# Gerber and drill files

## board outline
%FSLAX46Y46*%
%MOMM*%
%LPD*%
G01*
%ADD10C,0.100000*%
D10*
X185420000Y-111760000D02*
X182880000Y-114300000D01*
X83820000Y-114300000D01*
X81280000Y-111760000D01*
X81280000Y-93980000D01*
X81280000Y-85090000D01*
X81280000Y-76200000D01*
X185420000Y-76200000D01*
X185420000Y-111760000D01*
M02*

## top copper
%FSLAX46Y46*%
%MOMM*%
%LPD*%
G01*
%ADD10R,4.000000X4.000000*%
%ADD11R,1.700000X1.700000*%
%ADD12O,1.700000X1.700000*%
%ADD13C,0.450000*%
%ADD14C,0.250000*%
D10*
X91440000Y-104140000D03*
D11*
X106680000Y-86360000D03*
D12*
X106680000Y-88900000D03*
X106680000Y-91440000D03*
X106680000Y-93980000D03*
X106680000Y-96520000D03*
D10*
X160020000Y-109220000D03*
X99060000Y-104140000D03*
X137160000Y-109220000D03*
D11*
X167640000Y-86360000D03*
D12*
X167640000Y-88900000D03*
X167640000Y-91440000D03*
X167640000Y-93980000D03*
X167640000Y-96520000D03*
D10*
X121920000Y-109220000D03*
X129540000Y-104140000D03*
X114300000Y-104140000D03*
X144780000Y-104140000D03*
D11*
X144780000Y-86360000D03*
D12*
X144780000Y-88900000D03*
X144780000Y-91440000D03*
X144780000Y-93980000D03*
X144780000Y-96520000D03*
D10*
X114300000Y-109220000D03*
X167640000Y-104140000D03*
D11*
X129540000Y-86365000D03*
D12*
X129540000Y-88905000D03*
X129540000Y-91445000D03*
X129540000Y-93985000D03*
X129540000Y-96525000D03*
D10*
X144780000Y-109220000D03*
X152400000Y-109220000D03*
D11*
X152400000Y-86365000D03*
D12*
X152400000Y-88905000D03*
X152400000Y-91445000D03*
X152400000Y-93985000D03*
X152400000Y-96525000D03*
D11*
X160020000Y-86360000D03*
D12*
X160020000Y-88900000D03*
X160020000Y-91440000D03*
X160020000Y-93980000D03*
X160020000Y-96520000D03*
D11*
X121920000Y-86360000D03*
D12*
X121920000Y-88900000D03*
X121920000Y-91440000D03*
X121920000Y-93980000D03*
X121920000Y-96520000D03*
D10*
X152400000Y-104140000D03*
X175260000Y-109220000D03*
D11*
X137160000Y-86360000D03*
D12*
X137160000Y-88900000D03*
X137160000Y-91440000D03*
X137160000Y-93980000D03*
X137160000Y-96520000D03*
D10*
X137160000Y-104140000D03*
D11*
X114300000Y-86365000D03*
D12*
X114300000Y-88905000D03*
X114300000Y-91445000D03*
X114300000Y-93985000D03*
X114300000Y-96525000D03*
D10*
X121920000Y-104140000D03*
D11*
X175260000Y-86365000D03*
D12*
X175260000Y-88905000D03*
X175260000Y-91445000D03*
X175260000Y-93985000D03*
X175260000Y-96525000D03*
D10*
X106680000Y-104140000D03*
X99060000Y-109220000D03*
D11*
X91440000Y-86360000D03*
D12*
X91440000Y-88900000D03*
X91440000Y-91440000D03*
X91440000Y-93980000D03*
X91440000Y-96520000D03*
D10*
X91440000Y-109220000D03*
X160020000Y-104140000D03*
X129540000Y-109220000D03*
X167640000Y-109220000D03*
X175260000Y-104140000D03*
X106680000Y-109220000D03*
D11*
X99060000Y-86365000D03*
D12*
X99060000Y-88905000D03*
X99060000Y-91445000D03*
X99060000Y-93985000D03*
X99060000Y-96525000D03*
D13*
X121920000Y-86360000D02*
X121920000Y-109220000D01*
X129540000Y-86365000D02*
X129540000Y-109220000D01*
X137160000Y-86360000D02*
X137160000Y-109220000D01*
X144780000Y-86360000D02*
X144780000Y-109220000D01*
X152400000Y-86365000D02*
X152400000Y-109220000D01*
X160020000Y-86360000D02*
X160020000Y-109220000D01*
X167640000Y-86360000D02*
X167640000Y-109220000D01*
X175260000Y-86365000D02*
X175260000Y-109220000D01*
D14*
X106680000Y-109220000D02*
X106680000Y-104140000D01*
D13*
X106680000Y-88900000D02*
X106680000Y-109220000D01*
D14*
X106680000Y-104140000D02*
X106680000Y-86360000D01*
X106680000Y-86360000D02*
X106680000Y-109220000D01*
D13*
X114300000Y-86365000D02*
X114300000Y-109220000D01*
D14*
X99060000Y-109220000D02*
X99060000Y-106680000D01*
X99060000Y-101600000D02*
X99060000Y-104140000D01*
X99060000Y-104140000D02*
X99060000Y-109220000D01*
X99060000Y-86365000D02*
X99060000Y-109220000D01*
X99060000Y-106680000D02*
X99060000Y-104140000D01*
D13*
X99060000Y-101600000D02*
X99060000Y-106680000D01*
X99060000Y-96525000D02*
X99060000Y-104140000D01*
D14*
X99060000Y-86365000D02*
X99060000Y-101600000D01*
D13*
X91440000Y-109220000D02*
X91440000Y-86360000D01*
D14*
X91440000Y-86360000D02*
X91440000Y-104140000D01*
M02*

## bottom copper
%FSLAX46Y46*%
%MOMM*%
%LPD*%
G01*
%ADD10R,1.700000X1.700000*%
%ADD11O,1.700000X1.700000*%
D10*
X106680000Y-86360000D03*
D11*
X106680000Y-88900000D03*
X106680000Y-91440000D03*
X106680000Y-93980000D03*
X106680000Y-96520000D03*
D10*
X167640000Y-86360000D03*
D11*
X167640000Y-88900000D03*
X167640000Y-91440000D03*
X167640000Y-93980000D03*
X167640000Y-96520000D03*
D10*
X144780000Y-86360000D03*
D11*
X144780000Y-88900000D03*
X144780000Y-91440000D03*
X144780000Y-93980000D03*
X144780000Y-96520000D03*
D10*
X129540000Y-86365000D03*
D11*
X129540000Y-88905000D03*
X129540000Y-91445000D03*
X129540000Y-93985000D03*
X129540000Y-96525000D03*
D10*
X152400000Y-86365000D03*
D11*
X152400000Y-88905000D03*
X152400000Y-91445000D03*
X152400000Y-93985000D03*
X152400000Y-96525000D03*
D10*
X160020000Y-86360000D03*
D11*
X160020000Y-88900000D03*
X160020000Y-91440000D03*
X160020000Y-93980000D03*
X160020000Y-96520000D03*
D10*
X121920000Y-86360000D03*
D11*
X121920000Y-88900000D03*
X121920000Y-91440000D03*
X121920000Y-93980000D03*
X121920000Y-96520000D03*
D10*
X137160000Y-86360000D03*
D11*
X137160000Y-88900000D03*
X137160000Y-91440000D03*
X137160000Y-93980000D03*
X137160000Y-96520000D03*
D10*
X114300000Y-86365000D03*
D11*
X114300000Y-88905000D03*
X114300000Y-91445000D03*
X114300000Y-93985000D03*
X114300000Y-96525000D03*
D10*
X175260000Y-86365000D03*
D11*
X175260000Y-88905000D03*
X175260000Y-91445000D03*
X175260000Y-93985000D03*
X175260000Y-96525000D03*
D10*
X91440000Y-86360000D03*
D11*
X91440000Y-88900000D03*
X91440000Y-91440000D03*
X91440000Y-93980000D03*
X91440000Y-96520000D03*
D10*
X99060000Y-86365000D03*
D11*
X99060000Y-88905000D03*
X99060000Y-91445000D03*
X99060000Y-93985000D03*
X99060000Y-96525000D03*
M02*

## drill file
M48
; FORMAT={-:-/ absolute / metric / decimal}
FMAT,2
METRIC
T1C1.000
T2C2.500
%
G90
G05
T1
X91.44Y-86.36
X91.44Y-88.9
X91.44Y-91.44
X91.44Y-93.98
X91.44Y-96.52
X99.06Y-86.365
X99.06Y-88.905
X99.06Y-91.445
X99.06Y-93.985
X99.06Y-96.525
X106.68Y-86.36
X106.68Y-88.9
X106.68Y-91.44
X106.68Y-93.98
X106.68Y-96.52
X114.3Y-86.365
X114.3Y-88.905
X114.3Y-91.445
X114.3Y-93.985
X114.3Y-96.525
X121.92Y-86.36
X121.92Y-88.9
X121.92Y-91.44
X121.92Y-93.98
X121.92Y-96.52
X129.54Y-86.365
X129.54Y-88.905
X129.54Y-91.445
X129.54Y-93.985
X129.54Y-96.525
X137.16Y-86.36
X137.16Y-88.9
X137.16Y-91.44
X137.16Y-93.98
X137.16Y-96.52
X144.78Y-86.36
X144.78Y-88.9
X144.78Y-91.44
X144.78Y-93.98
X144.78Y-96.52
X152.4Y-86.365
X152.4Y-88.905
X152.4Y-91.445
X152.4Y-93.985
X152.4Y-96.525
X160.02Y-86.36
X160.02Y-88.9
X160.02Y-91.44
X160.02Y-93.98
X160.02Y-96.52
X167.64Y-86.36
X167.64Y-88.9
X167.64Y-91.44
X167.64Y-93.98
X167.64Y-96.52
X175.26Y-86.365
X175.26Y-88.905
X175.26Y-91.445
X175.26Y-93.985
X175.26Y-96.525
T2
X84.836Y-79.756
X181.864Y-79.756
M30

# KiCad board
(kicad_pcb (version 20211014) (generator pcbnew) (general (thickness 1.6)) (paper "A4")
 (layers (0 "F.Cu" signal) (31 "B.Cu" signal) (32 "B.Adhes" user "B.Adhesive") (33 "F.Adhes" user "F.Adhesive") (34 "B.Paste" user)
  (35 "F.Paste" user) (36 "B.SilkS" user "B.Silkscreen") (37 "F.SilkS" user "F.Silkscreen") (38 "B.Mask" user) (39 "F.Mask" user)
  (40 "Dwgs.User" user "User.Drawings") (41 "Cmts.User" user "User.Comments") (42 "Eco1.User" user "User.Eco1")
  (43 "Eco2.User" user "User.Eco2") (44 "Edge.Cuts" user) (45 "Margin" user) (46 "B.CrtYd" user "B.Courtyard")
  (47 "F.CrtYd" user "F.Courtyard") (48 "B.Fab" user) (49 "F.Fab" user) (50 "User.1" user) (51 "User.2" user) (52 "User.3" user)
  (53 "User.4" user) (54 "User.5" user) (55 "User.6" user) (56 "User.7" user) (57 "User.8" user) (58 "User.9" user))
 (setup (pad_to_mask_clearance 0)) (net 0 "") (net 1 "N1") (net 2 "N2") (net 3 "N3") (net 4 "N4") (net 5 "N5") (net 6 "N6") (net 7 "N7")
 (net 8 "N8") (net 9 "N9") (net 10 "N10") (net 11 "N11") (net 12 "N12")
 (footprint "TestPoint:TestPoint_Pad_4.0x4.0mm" (layer "F.Cu") (at 91.44 104.14 -90)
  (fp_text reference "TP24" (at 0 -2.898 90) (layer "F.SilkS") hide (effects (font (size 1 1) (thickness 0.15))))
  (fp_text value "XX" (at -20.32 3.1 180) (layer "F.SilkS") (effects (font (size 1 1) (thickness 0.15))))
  (pad "1" smd rect (at 0 0 270) (size 4 4) (layers "F.Cu" "F.Mask") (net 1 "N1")))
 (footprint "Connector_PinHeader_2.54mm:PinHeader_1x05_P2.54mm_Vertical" (layer "F.Cu") (at 106.68 86.36)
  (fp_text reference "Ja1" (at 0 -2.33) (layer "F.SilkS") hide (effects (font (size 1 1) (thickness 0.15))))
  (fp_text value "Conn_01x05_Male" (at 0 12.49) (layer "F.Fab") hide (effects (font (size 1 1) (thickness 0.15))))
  (pad "1" thru_hole rect (at 0 0) (size 1.7 1.7) (drill 1) (layers *.Cu *.Mask) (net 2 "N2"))
  (pad "2" thru_hole oval (at 0 2.54) (size 1.7 1.7) (drill 1) (layers *.Cu *.Mask) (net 2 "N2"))
  (pad "3" thru_hole oval (at 0 5.08) (size 1.7 1.7) (drill 1) (layers *.Cu *.Mask) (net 2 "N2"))
  (pad "4" thru_hole oval (at 0 7.62) (size 1.7 1.7) (drill 1) (layers *.Cu *.Mask) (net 2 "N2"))
  (pad "5" thru_hole oval (at 0 10.16) (size 1.7 1.7) (drill 1) (layers *.Cu *.Mask) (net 2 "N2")))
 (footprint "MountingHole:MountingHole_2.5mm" (layer "F.Cu") (at 84.836 79.756)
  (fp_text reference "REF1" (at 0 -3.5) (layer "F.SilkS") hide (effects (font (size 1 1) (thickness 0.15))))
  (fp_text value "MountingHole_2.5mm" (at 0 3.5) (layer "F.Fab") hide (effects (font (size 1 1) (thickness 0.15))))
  (pad "" np_thru_hole circle (at 0 0) (size 2.5 2.5) (drill 2.5) (layers *.Cu *.Mask)))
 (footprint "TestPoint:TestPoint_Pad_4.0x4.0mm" (layer "F.Cu") (at 160.02 109.22)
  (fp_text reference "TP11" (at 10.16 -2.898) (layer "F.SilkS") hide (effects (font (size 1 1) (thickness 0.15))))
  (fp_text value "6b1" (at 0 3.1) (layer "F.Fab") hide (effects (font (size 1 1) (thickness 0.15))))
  (pad "1" smd rect (at 0 0) (size 4 4) (layers "F.Cu" "F.Mask") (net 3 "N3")))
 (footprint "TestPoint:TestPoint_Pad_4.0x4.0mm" (layer "F.Cu") (at 99.06 104.14 -90)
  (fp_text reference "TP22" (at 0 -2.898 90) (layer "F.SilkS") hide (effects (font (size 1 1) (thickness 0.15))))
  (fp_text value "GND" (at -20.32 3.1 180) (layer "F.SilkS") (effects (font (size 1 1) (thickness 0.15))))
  (pad "1" smd rect (at 0 0 270) (size 4 4) (layers "F.Cu" "F.Mask") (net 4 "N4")))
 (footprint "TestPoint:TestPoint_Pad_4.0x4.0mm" (layer "F.Cu") (at 137.16 109.22)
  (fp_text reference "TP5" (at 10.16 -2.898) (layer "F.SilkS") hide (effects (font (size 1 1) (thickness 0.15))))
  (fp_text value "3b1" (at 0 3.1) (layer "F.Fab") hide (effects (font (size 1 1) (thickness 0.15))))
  (pad "1" smd rect (at 0 0) (size 4 4) (layers "F.Cu" "F.Mask") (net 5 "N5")))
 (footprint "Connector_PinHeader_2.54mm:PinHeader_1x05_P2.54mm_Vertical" (layer "F.Cu") (at 167.64 86.36)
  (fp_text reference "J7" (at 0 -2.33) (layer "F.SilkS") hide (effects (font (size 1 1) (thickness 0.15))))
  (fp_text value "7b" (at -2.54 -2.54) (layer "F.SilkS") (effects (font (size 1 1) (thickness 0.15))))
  (pad "1" thru_hole rect (at 0 0) (size 1.7 1.7) (drill 1) (layers *.Cu *.Mask) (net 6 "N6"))
  (pad "2" thru_hole oval (at 0 2.54) (size 1.7 1.7) (drill 1) (layers *.Cu *.Mask) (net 6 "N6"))
  (pad "3" thru_hole oval (at 0 5.08) (size 1.7 1.7) (drill 1) (layers *.Cu *.Mask) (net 6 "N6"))
  (pad "4" thru_hole oval (at 0 7.62) (size 1.7 1.7) (drill 1) (layers *.Cu *.Mask) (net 6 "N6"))
  (pad "5" thru_hole oval (at 0 10.16) (size 1.7 1.7) (drill 1) (layers *.Cu *.Mask) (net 6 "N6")))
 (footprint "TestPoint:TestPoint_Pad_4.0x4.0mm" (layer "F.Cu") (at 121.92 109.22)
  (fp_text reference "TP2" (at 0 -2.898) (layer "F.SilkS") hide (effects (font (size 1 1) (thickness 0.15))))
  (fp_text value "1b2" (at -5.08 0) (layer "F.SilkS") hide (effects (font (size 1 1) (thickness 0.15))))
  (pad "1" smd rect (at 0 0) (size 4 4) (layers "F.Cu" "F.Mask") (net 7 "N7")))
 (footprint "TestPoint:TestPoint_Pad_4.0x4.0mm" (layer "F.Cu") (at 129.54 104.14)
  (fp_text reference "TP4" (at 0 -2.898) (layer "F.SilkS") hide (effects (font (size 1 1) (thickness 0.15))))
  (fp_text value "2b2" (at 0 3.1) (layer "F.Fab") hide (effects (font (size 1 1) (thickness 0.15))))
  (pad "1" smd rect (at 0 0) (size 4 4) (layers "F.Cu" "F.Mask") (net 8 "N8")))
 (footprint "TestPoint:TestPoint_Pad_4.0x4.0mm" (layer "F.Cu") (at 114.3 104.14 -90)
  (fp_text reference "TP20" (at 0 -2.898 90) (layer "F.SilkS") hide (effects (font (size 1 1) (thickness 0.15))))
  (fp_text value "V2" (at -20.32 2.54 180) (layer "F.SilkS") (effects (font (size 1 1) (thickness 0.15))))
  (pad "1" smd rect (at 0 0 270) (size 4 4) (layers "F.Cu" "F.Mask") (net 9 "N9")))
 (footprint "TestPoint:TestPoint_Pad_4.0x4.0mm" (layer "F.Cu") (at 144.78 104.14)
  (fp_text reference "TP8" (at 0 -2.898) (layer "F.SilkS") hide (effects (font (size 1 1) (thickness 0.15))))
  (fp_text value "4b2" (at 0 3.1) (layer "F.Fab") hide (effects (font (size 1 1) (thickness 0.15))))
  (pad "1" smd rect (at 0 0) (size 4 4) (layers "F.Cu" "F.Mask") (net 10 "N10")))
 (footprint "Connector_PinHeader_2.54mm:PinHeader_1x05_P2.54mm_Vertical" (layer "F.Cu") (at 144.78 86.36)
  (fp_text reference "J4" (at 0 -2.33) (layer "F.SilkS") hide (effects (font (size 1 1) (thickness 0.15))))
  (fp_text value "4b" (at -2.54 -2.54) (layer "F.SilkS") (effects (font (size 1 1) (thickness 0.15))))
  (pad "1" thru_hole rect (at 0 0) (size 1.7 1.7) (drill 1) (layers *.Cu *.Mask) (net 10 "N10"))
  (pad "2" thru_hole oval (at 0 2.54) (size 1.7 1.7) (drill 1) (layers *.Cu *.Mask) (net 10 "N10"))
  (pad "3" thru_hole oval (at 0 5.08) (size 1.7 1.7) (drill 1) (layers *.Cu *.Mask) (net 10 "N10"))
  (pad "4" thru_hole oval (at 0 7.62) (size 1.7 1.7) (drill 1) (layers *.Cu *.Mask) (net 10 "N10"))
  (pad "5" thru_hole oval (at 0 10.16) (size 1.7 1.7) (drill 1) (layers *.Cu *.Mask) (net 10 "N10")))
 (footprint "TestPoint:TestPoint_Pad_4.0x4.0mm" (layer "F.Cu") (at 114.3 109.22 -90)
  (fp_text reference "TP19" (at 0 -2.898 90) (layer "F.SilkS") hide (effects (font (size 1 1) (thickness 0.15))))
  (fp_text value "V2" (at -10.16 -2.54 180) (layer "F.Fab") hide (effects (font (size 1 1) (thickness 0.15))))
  (pad "1" smd rect (at 0 0 270) (size 4 4) (layers "F.Cu" "F.Mask") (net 9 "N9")))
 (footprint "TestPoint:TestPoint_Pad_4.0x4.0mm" (layer "F.Cu") (at 167.64 104.14)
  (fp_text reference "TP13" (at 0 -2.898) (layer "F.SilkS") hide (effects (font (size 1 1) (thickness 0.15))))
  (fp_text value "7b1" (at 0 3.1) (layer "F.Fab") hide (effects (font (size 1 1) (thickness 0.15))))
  (pad "1" smd rect (at 0 0) (size 4 4) (layers "F.Cu" "F.Mask") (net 6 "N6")))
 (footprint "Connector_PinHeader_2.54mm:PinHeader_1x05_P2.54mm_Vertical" (layer "F.Cu") (at 129.54 86.365)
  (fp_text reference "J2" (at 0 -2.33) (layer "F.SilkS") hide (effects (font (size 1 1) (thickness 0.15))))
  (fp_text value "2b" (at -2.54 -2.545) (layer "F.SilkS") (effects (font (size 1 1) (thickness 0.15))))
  (pad "1" thru_hole rect (at 0 0) (size 1.7 1.7) (drill 1) (layers *.Cu *.Mask) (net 8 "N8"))
  (pad "2" thru_hole oval (at 0 2.54) (size 1.7 1.7) (drill 1) (layers *.Cu *.Mask) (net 8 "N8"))
  (pad "3" thru_hole oval (at 0 5.08) (size 1.7 1.7) (drill 1) (layers *.Cu *.Mask) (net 8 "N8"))
  (pad "4" thru_hole oval (at 0 7.62) (size 1.7 1.7) (drill 1) (layers *.Cu *.Mask) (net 8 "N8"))
  (pad "5" thru_hole oval (at 0 10.16) (size 1.7 1.7) (drill 1) (layers *.Cu *.Mask) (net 8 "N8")))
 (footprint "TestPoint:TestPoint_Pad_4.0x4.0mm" (layer "F.Cu") (at 144.78 109.22)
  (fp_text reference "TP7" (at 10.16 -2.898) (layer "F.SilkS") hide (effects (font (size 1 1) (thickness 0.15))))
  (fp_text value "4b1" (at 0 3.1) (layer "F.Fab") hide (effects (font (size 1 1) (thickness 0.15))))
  (pad "1" smd rect (at 0 0) (size 4 4) (layers "F.Cu" "F.Mask") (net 10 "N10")))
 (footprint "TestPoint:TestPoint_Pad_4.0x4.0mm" (layer "F.Cu") (at 152.4 109.22)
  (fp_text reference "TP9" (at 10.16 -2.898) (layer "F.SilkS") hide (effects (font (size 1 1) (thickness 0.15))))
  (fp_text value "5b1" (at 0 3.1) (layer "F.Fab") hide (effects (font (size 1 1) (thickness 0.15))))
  (pad "1" smd rect (at 0 0) (size 4 4) (layers "F.Cu" "F.Mask") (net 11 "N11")))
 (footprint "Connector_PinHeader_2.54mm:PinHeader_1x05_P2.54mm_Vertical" (layer "F.Cu") (at 152.4 86.365)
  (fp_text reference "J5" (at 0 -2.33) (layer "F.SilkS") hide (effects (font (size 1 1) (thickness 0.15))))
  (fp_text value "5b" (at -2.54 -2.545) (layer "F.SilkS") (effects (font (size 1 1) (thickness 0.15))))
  (pad "1" thru_hole rect (at 0 0) (size 1.7 1.7) (drill 1) (layers *.Cu *.Mask) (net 11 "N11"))
  (pad "2" thru_hole oval (at 0 2.54) (size 1.7 1.7) (drill 1) (layers *.Cu *.Mask) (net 11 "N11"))
  (pad "3" thru_hole oval (at 0 5.08) (size 1.7 1.7) (drill 1) (layers *.Cu *.Mask) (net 11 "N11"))
  (pad "4" thru_hole oval (at 0 7.62) (size 1.7 1.7) (drill 1) (layers *.Cu *.Mask) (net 11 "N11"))
  (pad "5" thru_hole oval (at 0 10.16) (size 1.7 1.7) (drill 1) (layers *.Cu *.Mask) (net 11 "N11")))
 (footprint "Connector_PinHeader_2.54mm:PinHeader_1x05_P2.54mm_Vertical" (layer "F.Cu") (at 160.02 86.36)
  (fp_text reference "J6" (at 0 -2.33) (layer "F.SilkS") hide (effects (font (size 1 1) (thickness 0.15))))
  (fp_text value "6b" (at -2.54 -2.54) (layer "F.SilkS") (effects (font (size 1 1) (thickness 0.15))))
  (pad "1" thru_hole rect (at 0 0) (size 1.7 1.7) (drill 1) (layers *.Cu *.Mask) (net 3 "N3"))
  (pad "2" thru_hole oval (at 0 2.54) (size 1.7 1.7) (drill 1) (layers *.Cu *.Mask) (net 3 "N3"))
  (pad "3" thru_hole oval (at 0 5.08) (size 1.7 1.7) (drill 1) (layers *.Cu *.Mask) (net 3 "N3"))
  (pad "4" thru_hole oval (at 0 7.62) (size 1.7 1.7) (drill 1) (layers *.Cu *.Mask) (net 3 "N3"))
  (pad "5" thru_hole oval (at 0 10.16) (size 1.7 1.7) (drill 1) (layers *.Cu *.Mask) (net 3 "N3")))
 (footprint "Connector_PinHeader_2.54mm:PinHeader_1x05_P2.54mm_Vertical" (layer "F.Cu") (at 121.92 86.36)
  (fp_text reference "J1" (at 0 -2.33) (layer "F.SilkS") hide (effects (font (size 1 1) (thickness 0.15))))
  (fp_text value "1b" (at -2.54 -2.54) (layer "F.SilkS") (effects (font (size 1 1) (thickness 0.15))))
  (pad "1" thru_hole rect (at 0 0) (size 1.7 1.7) (drill 1) (layers *.Cu *.Mask) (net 7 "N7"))
  (pad "2" thru_hole oval (at 0 2.54) (size 1.7 1.7) (drill 1) (layers *.Cu *.Mask) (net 7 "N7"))
  (pad "3" thru_hole oval (at 0 5.08) (size 1.7 1.7) (drill 1) (layers *.Cu *.Mask) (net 7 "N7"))
  (pad "4" thru_hole oval (at 0 7.62) (size 1.7 1.7) (drill 1) (layers *.Cu *.Mask) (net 7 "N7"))
  (pad "5" thru_hole oval (at 0 10.16) (size 1.7 1.7) (drill 1) (layers *.Cu *.Mask) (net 7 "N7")))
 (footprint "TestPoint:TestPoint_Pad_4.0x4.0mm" (layer "F.Cu") (at 152.4 104.14)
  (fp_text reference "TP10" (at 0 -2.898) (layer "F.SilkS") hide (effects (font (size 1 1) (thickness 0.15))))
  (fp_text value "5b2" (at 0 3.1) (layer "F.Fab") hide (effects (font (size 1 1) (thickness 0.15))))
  (pad "1" smd rect (at 0 0) (size 4 4) (layers "F.Cu" "F.Mask") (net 11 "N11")))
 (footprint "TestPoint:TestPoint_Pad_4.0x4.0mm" (layer "F.Cu") (at 175.26 109.22)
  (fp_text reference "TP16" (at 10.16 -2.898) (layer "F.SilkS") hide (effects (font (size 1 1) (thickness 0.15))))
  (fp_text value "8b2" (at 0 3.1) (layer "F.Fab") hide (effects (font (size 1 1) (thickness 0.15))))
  (pad "1" smd rect (at 0 0) (size 4 4) (layers "F.Cu" "F.Mask") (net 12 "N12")))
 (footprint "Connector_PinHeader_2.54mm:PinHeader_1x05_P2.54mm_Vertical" (layer "F.Cu") (at 137.16 86.36)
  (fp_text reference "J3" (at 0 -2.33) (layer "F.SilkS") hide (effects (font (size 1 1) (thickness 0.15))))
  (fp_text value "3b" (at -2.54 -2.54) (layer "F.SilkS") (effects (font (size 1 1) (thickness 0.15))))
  (pad "1" thru_hole rect (at 0 0) (size 1.7 1.7) (drill 1) (layers *.Cu *.Mask) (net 5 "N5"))
  (pad "2" thru_hole oval (at 0 2.54) (size 1.7 1.7) (drill 1) (layers *.Cu *.Mask) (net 5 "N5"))
  (pad "3" thru_hole oval (at 0 5.08) (size 1.7 1.7) (drill 1) (layers *.Cu *.Mask) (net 5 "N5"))
  (pad "4" thru_hole oval (at 0 7.62) (size 1.7 1.7) (drill 1) (layers *.Cu *.Mask) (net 5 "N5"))
  (pad "5" thru_hole oval (at 0 10.16) (size 1.7 1.7) (drill 1) (layers *.Cu *.Mask) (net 5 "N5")))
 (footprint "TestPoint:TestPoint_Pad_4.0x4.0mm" (layer "F.Cu") (at 137.16 104.14)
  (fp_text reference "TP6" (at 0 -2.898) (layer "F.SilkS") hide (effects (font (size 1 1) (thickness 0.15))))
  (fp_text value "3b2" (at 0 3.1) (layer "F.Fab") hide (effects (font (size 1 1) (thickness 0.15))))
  (pad "1" smd rect (at 0 0) (size 4 4) (layers "F.Cu" "F.Mask") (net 5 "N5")))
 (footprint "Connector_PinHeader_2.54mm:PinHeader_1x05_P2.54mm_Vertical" (layer "F.Cu") (at 114.3 86.365)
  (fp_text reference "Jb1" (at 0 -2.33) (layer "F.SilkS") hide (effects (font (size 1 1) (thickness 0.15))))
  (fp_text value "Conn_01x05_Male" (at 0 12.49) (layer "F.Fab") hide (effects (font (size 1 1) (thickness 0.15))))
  (pad "1" thru_hole rect (at 0 0) (size 1.7 1.7) (drill 1) (layers *.Cu *.Mask) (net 9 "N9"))
  (pad "2" thru_hole oval (at 0 2.54) (size 1.7 1.7) (drill 1) (layers *.Cu *.Mask) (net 9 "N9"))
  (pad "3" thru_hole oval (at 0 5.08) (size 1.7 1.7) (drill 1) (layers *.Cu *.Mask) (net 9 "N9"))
  (pad "4" thru_hole oval (at 0 7.62) (size 1.7 1.7) (drill 1) (layers *.Cu *.Mask) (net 9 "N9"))
  (pad "5" thru_hole oval (at 0 10.16) (size 1.7 1.7) (drill 1) (layers *.Cu *.Mask) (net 9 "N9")))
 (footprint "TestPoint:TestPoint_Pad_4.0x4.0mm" (layer "F.Cu") (at 121.92 104.14)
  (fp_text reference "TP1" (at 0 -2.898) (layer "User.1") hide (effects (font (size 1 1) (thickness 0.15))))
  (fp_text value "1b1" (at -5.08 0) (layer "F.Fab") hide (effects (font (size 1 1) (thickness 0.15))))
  (pad "1" smd rect (at 0 0) (size 4 4) (layers "F.Cu" "F.Mask") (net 7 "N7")))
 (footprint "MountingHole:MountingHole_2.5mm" (layer "F.Cu") (at 181.864 79.756)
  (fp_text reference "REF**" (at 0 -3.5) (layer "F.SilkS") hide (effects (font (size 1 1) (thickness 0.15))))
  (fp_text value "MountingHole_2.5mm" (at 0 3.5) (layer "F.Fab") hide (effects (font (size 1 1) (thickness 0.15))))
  (pad "" np_thru_hole circle (at 0 0) (size 2.5 2.5) (drill 2.5) (layers *.Cu *.Mask)))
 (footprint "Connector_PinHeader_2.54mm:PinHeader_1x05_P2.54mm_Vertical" (layer "F.Cu") (at 175.26 86.365)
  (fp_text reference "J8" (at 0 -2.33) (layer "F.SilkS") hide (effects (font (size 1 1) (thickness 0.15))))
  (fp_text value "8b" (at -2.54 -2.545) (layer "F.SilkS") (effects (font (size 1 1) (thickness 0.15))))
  (pad "1" thru_hole rect (at 0 0) (size 1.7 1.7) (drill 1) (layers *.Cu *.Mask) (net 12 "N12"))
  (pad "2" thru_hole oval (at 0 2.54) (size 1.7 1.7) (drill 1) (layers *.Cu *.Mask) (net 12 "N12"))
  (pad "3" thru_hole oval (at 0 5.08) (size 1.7 1.7) (drill 1) (layers *.Cu *.Mask) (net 12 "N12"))
  (pad "4" thru_hole oval (at 0 7.62) (size 1.7 1.7) (drill 1) (layers *.Cu *.Mask) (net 12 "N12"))
  (pad "5" thru_hole oval (at 0 10.16) (size 1.7 1.7) (drill 1) (layers *.Cu *.Mask) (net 12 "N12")))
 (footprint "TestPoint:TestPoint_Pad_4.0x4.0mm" (layer "F.Cu") (at 106.68 104.14 -90)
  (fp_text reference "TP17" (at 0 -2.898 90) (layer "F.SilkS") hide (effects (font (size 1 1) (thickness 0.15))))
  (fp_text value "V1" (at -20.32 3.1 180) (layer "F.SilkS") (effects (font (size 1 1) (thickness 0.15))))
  (pad "1" smd rect (at 0 0 270) (size 4 4) (layers "F.Cu" "F.Mask") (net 2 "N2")))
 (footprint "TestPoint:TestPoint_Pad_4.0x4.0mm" (layer "F.Cu") (at 99.06 109.22 -90)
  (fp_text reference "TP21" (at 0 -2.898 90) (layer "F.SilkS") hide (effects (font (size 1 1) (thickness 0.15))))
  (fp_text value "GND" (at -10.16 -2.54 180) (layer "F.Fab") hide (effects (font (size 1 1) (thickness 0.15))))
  (pad "1" smd rect (at 0 0 270) (size 4 4) (layers "F.Cu" "F.Mask") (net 4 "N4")))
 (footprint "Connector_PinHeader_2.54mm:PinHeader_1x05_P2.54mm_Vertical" (layer "F.Cu") (at 91.44 86.36)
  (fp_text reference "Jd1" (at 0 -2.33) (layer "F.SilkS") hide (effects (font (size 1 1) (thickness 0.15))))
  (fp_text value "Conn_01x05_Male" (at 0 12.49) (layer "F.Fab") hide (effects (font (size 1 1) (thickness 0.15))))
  (pad "1" thru_hole rect (at 0 0) (size 1.7 1.7) (drill 1) (layers *.Cu *.Mask) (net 1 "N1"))
  (pad "2" thru_hole oval (at 0 2.54) (size 1.7 1.7) (drill 1) (layers *.Cu *.Mask) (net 1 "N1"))
  (pad "3" thru_hole oval (at 0 5.08) (size 1.7 1.7) (drill 1) (layers *.Cu *.Mask) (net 1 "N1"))
  (pad "4" thru_hole oval (at 0 7.62) (size 1.7 1.7) (drill 1) (layers *.Cu *.Mask) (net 1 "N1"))
  (pad "5" thru_hole oval (at 0 10.16) (size 1.7 1.7) (drill 1) (layers *.Cu *.Mask) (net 1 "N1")))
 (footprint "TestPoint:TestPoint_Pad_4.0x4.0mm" (layer "F.Cu") (at 91.44 109.22 -90)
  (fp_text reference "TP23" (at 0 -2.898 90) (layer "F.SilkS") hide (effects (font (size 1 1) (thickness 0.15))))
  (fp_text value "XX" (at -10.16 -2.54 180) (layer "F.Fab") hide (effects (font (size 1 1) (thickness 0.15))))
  (pad "1" smd rect (at 0 0 270) (size 4 4) (layers "F.Cu" "F.Mask") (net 1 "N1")))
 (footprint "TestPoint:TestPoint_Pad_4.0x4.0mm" (layer "F.Cu") (at 160.02 104.14)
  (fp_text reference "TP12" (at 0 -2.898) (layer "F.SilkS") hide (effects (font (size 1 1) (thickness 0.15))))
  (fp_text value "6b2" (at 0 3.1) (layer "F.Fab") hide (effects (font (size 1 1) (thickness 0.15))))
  (pad "1" smd rect (at 0 0) (size 4 4) (layers "F.Cu" "F.Mask") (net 3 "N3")))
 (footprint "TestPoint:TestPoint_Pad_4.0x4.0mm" (layer "F.Cu") (at 129.54 109.22)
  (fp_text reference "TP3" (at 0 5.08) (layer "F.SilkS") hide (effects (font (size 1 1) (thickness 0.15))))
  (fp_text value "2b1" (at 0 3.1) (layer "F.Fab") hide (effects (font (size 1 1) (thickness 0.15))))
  (pad "1" smd rect (at 0 0) (size 4 4) (layers "F.Cu" "F.Mask") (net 8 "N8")))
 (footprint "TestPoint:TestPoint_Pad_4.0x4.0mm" (layer "F.Cu") (at 167.64 109.22)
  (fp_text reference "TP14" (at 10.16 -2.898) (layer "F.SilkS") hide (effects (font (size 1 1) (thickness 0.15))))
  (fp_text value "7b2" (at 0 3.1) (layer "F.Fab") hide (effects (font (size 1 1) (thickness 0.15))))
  (pad "1" smd rect (at 0 0) (size 4 4) (layers "F.Cu" "F.Mask") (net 6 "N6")))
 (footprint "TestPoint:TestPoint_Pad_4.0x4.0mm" (layer "F.Cu") (at 175.26 104.14)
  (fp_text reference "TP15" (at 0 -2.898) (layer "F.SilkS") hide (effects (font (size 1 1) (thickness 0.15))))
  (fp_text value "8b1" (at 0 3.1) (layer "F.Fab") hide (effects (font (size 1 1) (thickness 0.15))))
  (pad "1" smd rect (at 0 0) (size 4 4) (layers "F.Cu" "F.Mask") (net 12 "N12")))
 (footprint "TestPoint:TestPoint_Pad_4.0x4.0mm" (layer "F.Cu") (at 106.68 109.22 -90)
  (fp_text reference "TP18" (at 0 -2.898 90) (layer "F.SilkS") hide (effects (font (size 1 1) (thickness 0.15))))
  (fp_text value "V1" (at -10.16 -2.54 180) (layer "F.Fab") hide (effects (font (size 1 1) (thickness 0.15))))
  (pad "1" smd rect (at 0 0 270) (size 4 4) (layers "F.Cu" "F.Mask") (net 2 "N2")))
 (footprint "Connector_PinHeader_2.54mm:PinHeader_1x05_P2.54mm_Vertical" (layer "F.Cu") (at 99.06 86.365)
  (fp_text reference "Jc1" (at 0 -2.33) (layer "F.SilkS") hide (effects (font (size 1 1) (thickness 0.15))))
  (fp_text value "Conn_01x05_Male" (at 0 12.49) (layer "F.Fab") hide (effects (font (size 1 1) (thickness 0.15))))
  (pad "1" thru_hole rect (at 0 0) (size 1.7 1.7) (drill 1) (layers *.Cu *.Mask) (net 4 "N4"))
  (pad "2" thru_hole oval (at 0 2.54) (size 1.7 1.7) (drill 1) (layers *.Cu *.Mask) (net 4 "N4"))
  (pad "3" thru_hole oval (at 0 5.08) (size 1.7 1.7) (drill 1) (layers *.Cu *.Mask) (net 4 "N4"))
  (pad "4" thru_hole oval (at 0 7.62) (size 1.7 1.7) (drill 1) (layers *.Cu *.Mask) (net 4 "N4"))
  (pad "5" thru_hole oval (at 0 10.16) (size 1.7 1.7) (drill 1) (layers *.Cu *.Mask) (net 4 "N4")))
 (gr_poly
  (pts (xy 185.42 111.76) (xy 182.88 114.3) (xy 83.82 114.3) (xy 81.28 111.76) (xy 81.28 93.98) (xy 81.28 85.09) (xy 81.28 76.2)
   (xy 185.42 76.2))
  (layer "Edge.Cuts") (width 0.1) (fill none))
 (segment (start 121.92 86.36) (end 121.92 109.22) (width 0.45) (layer "F.Cu") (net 7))
 (segment (start 129.54 86.365) (end 129.54 109.22) (width 0.45) (layer "F.Cu") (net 8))
 (segment (start 137.16 86.36) (end 137.16 109.22) (width 0.45) (layer "F.Cu") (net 5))
 (segment (start 144.78 86.36) (end 144.78 109.22) (width 0.45) (layer "F.Cu") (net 10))
 (segment (start 152.4 86.365) (end 152.4 109.22) (width 0.45) (layer "F.Cu") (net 11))
 (segment (start 160.02 86.36) (end 160.02 109.22) (width 0.45) (layer "F.Cu") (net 3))
 (segment (start 167.64 86.36) (end 167.64 109.22) (width 0.45) (layer "F.Cu") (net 6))
 (segment (start 175.26 86.365) (end 175.26 109.22) (width 0.45) (layer "F.Cu") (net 12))
 (segment (start 106.68 109.22) (end 106.68 104.14) (width 0.25) (layer "F.Cu") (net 2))
 (segment (start 106.68 88.9) (end 106.68 109.22) (width 0.45) (layer "F.Cu") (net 2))
 (segment (start 106.68 104.14) (end 106.68 86.36) (width 0.25) (layer "F.Cu") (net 2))
 (segment (start 106.68 86.36) (end 106.68 109.22) (width 0.25) (layer "F.Cu") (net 2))
 (segment (start 114.3 86.365) (end 114.3 109.22) (width 0.45) (layer "F.Cu") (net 9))
 (segment (start 99.06 109.22) (end 99.06 106.68) (width 0.25) (layer "F.Cu") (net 4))
 (segment (start 99.06 101.6) (end 99.06 104.14) (width 0.25) (layer "F.Cu") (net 4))
 (segment (start 99.06 104.14) (end 99.06 109.22) (width 0.25) (layer "F.Cu") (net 4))
 (segment (start 99.06 86.365) (end 99.06 109.22) (width 0.25) (layer "F.Cu") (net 4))
 (segment (start 99.06 106.68) (end 99.06 104.14) (width 0.25) (layer "F.Cu") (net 4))
 (segment (start 99.06 101.6) (end 99.06 106.68) (width 0.45) (layer "F.Cu") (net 4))
 (segment (start 99.06 96.525) (end 99.06 104.14) (width 0.45) (layer "F.Cu") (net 4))
 (segment (start 99.06 86.365) (end 99.06 101.6) (width 0.25) (layer "F.Cu") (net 4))
 (segment (start 91.44 109.22) (end 91.44 86.36) (width 0.45) (layer "F.Cu") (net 1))
 (segment (start 91.44 86.36) (end 91.44 104.14) (width 0.25) (layer "F.Cu") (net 1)))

